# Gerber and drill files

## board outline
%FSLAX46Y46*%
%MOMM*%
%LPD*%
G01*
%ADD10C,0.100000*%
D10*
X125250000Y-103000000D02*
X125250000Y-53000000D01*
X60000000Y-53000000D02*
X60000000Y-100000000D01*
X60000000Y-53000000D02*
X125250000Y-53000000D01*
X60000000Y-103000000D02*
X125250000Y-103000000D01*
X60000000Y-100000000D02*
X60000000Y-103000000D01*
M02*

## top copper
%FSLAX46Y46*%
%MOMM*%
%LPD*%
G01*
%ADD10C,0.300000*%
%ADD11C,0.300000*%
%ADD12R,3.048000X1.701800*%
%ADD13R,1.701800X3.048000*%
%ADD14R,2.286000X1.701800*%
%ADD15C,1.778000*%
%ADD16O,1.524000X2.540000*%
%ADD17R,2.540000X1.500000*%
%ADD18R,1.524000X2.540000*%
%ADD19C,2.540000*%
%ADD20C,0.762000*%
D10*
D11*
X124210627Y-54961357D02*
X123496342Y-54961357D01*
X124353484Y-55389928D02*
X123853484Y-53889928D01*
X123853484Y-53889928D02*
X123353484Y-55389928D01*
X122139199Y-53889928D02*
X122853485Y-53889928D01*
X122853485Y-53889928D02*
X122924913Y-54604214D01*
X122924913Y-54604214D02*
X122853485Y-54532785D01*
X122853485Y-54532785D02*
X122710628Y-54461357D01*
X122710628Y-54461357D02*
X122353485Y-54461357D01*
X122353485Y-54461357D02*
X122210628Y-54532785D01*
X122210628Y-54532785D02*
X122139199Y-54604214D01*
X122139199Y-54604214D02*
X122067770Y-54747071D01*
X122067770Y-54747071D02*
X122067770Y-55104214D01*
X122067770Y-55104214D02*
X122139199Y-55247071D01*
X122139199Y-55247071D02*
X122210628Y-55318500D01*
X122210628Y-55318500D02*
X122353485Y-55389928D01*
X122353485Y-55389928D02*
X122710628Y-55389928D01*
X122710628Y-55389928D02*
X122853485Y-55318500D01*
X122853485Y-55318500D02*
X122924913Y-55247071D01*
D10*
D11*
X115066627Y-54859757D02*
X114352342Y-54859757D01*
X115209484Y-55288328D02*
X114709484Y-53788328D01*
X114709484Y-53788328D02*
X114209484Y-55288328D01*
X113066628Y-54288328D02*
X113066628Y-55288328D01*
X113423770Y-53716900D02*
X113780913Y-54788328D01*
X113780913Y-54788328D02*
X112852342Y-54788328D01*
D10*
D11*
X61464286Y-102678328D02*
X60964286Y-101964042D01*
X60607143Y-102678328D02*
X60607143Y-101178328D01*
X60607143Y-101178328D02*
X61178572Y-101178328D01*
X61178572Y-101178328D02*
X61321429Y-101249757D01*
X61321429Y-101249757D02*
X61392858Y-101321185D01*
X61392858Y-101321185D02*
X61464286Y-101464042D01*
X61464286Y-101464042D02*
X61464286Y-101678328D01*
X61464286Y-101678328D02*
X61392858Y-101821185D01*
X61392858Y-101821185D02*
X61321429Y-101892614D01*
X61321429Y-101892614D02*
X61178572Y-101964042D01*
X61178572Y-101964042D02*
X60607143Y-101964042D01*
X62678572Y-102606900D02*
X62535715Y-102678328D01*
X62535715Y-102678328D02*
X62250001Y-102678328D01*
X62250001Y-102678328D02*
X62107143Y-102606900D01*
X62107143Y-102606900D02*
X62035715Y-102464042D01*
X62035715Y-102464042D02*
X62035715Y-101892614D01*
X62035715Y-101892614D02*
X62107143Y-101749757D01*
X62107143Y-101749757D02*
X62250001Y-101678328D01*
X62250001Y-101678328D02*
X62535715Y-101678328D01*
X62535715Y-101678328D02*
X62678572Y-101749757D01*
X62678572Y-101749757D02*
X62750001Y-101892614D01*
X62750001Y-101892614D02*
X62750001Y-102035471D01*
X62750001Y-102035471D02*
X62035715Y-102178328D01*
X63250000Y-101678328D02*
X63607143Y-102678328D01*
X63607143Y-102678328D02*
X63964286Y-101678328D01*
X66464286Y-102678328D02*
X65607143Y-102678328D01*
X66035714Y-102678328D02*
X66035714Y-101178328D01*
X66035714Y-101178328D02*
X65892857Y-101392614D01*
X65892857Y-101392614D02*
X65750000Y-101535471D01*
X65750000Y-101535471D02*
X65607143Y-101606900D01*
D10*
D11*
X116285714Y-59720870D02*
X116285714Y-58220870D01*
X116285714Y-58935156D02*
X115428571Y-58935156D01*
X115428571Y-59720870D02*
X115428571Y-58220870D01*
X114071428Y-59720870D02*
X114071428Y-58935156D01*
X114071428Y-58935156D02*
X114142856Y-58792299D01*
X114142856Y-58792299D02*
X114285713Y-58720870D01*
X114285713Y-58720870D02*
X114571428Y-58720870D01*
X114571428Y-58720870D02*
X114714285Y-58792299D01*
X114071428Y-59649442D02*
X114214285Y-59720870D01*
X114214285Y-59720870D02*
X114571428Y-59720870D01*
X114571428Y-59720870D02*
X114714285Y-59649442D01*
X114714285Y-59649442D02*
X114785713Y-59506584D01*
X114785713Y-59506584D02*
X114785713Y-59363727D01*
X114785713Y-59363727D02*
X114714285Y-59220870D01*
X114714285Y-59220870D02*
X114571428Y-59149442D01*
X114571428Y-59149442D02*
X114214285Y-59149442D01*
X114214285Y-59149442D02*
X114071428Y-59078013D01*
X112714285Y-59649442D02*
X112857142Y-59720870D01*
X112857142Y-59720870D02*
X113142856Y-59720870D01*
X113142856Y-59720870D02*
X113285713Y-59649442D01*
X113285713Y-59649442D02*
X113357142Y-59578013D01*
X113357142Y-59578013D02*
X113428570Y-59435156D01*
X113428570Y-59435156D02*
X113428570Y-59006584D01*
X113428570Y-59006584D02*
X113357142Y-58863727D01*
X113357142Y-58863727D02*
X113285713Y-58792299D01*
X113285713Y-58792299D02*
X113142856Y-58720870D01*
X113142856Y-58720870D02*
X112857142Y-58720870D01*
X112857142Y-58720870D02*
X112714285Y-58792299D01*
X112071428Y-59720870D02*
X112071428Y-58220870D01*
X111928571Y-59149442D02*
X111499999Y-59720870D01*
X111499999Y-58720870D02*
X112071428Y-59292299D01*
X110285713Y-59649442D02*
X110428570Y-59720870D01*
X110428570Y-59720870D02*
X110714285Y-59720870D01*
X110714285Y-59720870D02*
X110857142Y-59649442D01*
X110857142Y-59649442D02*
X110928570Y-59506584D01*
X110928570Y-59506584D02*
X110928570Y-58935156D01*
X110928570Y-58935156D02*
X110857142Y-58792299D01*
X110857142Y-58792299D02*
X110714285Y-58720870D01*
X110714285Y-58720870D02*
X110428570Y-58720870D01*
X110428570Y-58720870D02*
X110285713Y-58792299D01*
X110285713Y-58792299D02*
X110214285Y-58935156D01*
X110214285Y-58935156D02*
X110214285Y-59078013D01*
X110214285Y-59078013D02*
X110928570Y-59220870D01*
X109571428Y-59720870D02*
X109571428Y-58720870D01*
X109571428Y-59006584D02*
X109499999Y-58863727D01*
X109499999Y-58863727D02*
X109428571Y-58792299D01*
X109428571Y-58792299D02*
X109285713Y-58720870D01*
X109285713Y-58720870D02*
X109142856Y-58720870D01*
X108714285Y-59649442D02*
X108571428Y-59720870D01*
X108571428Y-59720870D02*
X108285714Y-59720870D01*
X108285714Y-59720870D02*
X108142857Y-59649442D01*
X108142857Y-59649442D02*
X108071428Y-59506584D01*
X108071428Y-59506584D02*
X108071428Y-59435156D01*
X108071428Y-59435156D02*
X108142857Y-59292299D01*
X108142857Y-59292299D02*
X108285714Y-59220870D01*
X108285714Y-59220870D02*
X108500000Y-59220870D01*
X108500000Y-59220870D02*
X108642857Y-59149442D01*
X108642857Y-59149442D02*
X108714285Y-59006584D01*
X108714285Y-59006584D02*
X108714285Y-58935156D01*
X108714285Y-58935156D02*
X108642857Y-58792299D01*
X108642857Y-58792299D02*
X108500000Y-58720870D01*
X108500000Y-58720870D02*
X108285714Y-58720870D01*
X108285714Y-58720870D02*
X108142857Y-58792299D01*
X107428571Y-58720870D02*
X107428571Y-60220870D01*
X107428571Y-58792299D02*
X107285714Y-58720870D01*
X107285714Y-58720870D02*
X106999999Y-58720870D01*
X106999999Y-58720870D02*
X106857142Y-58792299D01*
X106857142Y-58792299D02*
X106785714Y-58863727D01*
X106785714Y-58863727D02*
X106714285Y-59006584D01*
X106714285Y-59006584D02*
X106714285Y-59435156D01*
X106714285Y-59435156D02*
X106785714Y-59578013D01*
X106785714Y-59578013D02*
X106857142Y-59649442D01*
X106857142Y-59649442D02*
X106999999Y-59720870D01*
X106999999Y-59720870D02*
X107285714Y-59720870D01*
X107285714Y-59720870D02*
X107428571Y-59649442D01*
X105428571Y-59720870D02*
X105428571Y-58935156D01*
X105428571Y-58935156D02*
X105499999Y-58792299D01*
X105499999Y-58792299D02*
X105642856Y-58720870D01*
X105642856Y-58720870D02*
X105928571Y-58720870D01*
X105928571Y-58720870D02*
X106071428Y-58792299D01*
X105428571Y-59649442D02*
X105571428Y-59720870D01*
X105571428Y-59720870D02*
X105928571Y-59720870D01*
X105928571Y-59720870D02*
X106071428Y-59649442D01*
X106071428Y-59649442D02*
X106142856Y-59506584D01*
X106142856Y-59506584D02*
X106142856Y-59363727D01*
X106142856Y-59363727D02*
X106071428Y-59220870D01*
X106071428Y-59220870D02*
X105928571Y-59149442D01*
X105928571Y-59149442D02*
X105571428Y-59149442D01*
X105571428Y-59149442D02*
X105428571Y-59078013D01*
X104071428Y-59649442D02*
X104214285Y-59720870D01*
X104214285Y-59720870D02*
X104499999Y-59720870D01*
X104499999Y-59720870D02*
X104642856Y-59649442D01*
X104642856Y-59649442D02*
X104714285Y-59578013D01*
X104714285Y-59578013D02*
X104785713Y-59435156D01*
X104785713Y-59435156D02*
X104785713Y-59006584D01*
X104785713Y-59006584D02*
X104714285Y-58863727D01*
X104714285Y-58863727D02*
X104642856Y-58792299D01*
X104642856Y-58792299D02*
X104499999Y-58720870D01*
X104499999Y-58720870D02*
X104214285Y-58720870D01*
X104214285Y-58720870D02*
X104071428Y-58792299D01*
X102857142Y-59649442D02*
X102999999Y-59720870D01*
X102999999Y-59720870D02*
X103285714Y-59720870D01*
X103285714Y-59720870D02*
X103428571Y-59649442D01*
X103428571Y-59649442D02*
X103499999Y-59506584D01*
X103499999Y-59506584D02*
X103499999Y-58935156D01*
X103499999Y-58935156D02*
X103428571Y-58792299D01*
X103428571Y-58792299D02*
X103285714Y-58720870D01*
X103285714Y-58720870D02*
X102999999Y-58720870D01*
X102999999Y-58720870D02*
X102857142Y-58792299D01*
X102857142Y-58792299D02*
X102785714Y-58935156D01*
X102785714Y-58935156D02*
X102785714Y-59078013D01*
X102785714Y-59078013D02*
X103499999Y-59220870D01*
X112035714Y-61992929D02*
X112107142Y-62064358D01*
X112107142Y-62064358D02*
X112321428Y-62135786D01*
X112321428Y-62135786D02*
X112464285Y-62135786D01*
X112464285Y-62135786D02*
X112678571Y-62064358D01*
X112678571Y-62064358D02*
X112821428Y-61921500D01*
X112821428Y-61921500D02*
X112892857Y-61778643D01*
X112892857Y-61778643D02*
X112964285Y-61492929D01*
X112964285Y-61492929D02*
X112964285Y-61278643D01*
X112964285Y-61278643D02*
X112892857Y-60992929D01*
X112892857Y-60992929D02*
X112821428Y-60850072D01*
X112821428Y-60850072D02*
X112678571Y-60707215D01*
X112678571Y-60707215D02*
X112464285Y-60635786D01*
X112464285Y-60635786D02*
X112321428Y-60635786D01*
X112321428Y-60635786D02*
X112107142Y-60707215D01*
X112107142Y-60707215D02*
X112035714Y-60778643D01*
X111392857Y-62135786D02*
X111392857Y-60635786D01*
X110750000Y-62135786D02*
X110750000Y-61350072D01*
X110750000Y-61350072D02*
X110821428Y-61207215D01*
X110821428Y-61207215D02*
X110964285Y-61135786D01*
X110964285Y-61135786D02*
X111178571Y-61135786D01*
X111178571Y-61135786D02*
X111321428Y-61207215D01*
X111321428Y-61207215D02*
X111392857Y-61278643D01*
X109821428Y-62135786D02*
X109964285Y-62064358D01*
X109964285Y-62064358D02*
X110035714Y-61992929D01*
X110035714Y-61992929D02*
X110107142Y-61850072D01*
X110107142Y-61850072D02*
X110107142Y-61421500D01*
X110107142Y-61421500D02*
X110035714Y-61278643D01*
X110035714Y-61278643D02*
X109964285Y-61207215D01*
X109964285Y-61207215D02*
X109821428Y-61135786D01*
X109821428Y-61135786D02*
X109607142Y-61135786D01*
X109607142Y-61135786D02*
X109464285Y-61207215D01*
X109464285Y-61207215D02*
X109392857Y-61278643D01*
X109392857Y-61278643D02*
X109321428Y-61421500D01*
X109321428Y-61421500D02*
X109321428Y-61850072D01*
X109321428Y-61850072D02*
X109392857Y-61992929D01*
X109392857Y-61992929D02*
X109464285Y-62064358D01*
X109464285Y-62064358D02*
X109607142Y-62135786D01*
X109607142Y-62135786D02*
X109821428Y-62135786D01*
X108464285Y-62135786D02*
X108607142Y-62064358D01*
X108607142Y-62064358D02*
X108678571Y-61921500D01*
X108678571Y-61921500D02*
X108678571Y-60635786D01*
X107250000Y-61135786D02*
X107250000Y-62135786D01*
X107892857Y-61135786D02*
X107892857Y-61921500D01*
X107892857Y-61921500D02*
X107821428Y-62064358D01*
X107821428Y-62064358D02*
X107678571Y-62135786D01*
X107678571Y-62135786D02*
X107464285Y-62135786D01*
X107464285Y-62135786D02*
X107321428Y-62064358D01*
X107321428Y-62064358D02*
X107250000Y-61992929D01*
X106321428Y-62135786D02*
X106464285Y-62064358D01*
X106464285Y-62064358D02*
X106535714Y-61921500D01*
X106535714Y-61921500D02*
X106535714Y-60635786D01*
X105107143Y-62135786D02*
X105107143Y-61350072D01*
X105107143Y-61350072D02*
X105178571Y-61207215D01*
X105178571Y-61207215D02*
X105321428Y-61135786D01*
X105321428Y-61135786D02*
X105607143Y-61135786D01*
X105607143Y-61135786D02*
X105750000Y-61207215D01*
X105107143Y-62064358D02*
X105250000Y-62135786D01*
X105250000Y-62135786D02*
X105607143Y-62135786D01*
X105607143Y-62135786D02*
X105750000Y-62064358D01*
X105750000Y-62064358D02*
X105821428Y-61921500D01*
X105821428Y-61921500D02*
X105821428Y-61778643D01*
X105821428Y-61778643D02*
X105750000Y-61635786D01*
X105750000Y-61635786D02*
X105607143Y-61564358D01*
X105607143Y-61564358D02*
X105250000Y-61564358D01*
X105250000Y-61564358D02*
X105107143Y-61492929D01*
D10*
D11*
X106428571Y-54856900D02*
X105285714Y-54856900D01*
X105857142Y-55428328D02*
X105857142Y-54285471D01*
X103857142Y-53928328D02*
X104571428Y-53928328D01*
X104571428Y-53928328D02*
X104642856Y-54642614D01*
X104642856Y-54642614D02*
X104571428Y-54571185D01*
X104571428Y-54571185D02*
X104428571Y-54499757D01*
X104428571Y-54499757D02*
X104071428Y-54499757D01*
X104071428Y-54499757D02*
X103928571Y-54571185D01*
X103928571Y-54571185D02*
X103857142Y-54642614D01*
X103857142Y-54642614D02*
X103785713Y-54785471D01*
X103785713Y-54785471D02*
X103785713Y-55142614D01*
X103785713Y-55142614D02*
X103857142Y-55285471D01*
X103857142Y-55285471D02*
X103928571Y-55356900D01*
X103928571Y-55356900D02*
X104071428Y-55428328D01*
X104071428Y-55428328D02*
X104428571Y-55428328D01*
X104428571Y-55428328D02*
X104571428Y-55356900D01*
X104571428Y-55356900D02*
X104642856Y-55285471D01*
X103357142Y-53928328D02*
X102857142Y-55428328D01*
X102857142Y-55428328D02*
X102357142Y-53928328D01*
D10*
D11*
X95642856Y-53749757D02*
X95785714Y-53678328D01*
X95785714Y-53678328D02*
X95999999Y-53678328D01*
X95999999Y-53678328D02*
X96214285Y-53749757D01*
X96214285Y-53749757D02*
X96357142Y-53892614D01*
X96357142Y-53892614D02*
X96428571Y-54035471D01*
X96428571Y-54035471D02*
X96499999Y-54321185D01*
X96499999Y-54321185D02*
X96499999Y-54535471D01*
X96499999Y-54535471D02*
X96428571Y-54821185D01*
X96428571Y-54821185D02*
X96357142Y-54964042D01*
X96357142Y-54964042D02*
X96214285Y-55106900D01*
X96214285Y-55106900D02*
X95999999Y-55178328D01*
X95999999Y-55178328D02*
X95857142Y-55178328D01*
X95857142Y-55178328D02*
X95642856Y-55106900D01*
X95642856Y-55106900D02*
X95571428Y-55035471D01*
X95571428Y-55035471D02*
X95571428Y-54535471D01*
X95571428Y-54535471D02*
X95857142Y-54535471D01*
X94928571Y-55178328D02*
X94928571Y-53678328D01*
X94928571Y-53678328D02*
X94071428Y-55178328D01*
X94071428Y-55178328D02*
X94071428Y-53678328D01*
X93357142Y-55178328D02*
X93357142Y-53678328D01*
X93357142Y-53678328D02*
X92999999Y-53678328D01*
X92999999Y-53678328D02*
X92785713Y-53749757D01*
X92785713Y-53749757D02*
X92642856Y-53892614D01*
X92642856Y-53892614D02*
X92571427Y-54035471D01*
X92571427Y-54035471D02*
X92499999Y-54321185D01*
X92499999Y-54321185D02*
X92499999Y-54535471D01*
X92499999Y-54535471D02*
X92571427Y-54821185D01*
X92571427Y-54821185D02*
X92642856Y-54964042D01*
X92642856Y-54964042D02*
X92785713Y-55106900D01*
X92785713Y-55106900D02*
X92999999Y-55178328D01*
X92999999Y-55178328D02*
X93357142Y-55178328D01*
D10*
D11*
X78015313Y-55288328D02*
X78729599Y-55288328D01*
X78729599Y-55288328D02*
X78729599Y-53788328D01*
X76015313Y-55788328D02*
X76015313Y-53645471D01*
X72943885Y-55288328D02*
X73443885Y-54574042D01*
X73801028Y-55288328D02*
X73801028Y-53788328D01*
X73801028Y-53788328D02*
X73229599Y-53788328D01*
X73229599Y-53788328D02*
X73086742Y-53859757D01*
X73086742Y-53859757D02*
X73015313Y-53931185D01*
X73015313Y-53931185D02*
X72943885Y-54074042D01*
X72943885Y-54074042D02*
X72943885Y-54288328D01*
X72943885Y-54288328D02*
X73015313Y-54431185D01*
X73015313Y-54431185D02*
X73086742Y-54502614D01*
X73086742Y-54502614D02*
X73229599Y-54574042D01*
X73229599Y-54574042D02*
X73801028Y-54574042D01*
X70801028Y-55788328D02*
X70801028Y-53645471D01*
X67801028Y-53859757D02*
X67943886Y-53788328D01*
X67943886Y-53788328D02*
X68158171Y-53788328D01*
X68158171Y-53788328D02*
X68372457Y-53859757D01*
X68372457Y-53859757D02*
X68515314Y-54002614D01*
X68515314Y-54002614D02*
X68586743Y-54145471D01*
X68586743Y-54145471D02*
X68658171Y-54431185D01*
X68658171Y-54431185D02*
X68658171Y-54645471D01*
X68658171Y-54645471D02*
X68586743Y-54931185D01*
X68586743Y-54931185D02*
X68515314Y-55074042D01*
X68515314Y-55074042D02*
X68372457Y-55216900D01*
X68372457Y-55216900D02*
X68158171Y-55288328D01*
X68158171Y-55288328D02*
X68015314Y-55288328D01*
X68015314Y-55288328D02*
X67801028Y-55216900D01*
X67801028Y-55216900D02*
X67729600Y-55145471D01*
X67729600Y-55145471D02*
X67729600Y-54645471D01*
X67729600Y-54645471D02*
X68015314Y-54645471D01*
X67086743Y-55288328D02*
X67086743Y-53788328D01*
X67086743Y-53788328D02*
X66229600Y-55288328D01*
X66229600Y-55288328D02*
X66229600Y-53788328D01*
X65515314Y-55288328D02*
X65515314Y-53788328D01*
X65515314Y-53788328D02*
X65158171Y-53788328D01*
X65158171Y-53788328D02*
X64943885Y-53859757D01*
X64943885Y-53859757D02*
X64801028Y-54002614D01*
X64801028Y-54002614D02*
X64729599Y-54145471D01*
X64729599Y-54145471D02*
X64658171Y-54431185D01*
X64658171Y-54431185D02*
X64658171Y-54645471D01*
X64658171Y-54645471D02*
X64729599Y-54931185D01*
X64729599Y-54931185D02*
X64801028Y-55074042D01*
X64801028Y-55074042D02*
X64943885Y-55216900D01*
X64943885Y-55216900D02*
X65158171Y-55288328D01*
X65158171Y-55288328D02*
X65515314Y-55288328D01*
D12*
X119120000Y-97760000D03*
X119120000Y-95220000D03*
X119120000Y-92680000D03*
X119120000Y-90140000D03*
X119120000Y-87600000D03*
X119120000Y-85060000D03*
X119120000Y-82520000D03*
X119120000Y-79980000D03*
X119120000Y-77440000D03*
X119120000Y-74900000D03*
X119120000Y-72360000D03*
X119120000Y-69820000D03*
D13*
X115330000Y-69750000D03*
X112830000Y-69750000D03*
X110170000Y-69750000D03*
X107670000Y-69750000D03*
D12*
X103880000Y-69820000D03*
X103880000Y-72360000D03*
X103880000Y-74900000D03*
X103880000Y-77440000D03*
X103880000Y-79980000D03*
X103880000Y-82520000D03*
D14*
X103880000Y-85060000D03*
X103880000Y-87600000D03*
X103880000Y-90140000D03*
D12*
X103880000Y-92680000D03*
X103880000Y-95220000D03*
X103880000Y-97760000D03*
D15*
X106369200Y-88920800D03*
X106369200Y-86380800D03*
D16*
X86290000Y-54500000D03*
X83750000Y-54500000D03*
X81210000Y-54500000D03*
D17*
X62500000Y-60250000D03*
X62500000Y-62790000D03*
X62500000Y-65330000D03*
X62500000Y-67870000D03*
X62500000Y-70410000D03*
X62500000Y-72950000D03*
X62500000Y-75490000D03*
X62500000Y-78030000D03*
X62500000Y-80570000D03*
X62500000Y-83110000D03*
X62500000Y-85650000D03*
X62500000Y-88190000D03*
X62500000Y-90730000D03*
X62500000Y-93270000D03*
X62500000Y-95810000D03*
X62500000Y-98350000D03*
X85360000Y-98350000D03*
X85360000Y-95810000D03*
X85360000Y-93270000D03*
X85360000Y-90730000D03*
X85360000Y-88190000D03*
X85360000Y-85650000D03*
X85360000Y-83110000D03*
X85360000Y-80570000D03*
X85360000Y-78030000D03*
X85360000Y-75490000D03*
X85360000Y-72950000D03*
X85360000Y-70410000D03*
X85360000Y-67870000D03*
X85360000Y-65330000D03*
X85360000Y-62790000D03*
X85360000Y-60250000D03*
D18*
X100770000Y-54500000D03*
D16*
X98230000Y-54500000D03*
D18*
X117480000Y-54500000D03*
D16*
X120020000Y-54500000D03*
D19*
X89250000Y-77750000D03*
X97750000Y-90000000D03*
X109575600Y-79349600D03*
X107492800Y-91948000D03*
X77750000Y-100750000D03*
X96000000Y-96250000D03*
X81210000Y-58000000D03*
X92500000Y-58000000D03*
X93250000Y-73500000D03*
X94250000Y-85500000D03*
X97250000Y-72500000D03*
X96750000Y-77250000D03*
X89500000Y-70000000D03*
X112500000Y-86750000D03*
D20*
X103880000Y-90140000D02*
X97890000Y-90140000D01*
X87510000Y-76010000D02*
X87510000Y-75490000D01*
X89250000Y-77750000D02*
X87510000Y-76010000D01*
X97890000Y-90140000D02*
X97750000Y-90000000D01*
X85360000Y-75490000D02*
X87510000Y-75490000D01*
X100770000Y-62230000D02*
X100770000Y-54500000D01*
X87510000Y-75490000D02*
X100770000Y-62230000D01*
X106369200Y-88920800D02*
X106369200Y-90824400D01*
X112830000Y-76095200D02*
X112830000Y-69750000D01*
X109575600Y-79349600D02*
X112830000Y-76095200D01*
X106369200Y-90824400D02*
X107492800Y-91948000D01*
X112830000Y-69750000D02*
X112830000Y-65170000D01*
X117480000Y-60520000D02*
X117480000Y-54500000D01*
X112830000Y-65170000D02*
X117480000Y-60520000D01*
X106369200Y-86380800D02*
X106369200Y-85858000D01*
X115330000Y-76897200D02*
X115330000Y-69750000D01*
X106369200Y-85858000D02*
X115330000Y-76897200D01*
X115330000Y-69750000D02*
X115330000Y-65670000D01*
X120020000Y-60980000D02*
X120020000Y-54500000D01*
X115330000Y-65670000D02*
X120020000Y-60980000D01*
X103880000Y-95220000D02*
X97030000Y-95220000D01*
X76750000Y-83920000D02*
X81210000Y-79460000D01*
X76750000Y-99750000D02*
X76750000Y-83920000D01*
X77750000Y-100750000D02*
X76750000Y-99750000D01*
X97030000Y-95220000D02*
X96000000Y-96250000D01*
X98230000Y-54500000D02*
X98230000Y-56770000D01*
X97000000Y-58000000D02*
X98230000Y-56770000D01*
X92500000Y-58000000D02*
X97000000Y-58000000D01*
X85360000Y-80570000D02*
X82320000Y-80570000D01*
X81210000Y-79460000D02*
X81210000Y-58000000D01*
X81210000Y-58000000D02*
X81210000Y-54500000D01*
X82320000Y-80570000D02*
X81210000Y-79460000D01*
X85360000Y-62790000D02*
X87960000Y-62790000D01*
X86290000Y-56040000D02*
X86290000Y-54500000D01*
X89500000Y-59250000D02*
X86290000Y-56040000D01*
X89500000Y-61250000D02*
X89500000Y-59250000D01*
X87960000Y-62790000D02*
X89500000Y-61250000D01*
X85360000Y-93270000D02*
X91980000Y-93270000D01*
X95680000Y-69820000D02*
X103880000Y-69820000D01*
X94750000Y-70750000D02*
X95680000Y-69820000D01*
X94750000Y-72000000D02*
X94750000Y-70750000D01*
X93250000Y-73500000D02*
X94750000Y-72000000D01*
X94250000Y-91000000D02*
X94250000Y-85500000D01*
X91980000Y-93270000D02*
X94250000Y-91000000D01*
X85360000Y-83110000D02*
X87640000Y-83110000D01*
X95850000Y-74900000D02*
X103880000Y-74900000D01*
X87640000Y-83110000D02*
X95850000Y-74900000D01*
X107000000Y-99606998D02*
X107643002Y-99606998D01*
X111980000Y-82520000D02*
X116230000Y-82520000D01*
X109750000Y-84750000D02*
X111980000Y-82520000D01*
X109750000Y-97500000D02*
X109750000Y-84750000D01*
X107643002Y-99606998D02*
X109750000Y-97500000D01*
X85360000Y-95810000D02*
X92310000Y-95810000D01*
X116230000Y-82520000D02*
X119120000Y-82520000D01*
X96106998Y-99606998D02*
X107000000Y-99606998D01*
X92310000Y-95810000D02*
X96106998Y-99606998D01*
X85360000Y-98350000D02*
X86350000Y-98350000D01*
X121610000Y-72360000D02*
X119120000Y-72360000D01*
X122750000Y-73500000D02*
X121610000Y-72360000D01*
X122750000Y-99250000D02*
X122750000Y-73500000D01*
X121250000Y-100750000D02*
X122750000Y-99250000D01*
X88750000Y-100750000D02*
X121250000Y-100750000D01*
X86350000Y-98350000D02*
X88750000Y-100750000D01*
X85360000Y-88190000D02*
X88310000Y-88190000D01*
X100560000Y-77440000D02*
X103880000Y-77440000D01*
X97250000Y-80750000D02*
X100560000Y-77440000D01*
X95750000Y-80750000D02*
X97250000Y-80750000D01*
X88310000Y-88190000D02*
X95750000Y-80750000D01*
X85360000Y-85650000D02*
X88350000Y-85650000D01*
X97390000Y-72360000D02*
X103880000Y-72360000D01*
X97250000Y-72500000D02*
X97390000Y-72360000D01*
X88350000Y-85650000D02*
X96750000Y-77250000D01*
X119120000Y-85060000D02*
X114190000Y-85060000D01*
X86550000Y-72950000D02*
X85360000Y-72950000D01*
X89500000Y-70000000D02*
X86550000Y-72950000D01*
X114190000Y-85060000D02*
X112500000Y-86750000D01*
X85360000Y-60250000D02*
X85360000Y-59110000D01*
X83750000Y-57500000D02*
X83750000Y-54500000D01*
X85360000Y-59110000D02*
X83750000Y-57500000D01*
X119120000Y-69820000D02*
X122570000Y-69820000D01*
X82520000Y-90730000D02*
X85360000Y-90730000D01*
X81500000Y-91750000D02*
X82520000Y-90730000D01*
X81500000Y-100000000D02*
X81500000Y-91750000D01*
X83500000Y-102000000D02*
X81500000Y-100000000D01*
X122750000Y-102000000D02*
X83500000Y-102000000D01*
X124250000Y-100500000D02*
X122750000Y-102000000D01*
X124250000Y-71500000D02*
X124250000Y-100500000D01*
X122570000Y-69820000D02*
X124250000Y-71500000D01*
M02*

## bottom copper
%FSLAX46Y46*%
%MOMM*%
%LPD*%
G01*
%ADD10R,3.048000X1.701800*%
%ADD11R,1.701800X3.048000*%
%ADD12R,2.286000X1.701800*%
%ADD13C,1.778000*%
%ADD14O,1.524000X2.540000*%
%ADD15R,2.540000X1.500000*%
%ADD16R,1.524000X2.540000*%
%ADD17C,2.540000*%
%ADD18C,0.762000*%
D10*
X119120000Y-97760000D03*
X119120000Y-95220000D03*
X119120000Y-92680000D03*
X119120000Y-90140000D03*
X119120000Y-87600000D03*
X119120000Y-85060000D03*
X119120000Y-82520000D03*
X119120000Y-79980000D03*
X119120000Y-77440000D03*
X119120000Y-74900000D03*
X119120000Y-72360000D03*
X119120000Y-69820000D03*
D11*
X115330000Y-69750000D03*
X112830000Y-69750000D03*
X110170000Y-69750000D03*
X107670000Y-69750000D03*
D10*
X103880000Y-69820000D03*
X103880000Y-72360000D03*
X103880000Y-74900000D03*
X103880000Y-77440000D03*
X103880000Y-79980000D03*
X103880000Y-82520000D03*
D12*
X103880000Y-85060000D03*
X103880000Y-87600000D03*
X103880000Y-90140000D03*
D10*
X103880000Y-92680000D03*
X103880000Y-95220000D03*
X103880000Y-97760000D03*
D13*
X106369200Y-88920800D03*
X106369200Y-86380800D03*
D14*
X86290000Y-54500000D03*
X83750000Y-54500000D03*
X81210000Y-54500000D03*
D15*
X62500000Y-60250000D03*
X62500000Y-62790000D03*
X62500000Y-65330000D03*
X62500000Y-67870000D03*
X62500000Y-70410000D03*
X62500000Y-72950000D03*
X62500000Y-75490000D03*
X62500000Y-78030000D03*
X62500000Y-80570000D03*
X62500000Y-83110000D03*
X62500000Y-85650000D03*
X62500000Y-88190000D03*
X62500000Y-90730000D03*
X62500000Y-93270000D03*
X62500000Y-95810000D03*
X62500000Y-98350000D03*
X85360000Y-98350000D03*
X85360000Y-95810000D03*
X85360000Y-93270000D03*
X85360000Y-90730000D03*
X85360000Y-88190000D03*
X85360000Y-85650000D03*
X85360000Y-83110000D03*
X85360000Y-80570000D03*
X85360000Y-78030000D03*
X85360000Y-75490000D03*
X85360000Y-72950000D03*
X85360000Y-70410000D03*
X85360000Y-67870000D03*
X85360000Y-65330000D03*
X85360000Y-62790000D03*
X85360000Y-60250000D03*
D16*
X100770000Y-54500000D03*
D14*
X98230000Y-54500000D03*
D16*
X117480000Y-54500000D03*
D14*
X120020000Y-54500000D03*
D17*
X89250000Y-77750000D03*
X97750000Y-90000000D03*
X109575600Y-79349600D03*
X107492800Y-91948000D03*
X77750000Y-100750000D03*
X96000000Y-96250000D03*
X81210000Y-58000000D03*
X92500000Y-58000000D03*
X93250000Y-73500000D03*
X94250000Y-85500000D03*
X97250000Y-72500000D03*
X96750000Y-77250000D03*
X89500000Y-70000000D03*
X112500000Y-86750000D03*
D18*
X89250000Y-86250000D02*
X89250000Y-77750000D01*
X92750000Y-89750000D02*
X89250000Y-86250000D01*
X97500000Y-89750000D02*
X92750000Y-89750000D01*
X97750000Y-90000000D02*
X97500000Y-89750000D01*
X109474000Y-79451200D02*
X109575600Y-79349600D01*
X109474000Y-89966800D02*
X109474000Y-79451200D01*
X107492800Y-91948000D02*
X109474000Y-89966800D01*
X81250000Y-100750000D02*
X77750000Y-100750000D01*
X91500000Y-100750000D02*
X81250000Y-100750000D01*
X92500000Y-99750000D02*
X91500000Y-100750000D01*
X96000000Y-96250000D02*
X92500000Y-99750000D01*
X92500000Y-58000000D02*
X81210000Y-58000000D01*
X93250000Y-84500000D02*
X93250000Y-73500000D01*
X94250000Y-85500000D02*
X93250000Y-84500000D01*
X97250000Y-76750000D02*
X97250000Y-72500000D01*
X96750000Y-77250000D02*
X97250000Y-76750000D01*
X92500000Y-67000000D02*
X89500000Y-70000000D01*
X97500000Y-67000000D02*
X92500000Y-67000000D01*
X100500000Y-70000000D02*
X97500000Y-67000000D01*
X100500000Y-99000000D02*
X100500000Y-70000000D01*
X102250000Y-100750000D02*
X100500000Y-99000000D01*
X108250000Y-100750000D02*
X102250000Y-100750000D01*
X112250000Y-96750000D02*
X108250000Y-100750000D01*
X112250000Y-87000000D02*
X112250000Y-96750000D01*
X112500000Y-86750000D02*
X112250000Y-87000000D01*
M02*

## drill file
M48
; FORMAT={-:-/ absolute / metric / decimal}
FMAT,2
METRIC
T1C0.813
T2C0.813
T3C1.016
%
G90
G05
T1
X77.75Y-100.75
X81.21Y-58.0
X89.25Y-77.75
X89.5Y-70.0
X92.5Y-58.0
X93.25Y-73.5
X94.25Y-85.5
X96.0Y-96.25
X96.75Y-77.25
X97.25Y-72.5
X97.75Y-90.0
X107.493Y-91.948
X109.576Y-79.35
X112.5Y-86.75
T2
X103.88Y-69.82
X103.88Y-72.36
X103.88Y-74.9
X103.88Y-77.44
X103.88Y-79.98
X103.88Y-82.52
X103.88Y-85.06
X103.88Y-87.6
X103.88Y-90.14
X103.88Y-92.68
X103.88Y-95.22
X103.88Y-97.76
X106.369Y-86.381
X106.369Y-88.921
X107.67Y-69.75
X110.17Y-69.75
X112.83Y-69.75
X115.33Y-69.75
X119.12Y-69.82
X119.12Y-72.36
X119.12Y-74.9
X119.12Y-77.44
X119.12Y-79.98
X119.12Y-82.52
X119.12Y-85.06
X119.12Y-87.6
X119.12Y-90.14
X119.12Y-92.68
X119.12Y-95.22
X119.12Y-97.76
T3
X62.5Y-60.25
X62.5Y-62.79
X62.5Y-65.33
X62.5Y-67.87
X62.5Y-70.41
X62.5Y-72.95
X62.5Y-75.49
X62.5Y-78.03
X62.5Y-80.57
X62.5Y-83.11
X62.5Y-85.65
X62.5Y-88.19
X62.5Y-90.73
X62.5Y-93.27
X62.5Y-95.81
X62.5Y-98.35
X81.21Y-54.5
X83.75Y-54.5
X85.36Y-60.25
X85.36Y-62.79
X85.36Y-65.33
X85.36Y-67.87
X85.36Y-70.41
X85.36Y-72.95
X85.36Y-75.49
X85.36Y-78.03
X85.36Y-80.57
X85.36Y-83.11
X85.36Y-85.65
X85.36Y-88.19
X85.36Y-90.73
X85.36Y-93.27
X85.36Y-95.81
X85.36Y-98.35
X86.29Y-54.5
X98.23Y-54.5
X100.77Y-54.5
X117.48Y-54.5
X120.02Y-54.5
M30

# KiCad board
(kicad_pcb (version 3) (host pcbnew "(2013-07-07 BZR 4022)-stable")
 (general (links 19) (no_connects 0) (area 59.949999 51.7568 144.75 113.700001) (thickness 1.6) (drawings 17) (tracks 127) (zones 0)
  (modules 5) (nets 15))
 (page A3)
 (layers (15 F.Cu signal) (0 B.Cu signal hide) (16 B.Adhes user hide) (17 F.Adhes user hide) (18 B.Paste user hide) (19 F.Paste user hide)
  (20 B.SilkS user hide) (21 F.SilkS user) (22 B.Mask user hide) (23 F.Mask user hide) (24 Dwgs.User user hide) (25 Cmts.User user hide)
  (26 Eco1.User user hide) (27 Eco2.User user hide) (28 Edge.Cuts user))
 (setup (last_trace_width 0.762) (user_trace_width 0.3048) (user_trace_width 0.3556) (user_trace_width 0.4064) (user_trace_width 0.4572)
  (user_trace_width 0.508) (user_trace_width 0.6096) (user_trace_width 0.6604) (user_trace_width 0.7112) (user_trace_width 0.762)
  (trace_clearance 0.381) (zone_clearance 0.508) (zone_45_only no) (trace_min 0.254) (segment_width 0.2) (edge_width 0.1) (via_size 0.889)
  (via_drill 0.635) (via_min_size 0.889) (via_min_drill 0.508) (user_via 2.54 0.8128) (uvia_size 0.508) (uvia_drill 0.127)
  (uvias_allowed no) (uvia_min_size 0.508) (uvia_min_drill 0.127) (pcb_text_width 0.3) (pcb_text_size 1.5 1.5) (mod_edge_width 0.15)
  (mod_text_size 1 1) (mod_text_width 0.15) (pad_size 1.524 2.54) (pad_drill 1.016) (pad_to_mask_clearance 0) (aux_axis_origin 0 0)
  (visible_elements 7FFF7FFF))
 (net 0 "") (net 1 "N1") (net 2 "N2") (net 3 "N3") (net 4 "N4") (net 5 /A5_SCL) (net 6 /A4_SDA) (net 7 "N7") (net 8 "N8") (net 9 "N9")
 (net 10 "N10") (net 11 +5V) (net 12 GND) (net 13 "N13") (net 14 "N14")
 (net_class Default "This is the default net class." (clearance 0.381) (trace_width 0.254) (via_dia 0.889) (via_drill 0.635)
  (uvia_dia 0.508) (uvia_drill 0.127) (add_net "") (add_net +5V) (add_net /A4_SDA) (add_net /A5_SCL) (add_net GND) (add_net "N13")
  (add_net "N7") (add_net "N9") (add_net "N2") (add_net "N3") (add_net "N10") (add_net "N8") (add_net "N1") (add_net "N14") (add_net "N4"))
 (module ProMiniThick (layer F.Cu) (at 111.5 81.25 90)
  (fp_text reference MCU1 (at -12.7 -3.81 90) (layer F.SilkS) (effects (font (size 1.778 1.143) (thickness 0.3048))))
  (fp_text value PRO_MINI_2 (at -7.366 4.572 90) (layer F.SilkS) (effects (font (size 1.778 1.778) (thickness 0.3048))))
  (pad 1 thru_hole rect (at -16.51 7.62 90) (size 1.7018 3.048) (drill 0.8128) (layers *.Cu *.Mask F.SilkS))
  (pad 2 thru_hole rect (at -13.97 7.62 90) (size 1.7018 3.048) (drill 0.8128) (layers *.Cu *.Mask F.SilkS))
  (pad 3 thru_hole rect (at -11.43 7.62 90) (size 1.7018 3.048) (drill 0.8128) (layers *.Cu *.Mask F.SilkS))
  (pad 4 thru_hole rect (at -8.89 7.62 90) (size 1.7018 3.048) (drill 0.8128) (layers *.Cu *.Mask F.SilkS))
  (pad 5 thru_hole rect (at -6.35 7.62 90) (size 1.7018 3.048) (drill 0.8128) (layers *.Cu *.Mask F.SilkS))
  (pad 6 thru_hole rect (at -3.81 7.62 90) (size 1.7018 3.048) (drill 0.8128) (layers *.Cu *.Mask F.SilkS) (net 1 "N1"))
  (pad 7 thru_hole rect (at -1.27 7.62 90) (size 1.7018 3.048) (drill 0.8128) (layers *.Cu *.Mask F.SilkS) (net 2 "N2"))
  (pad 8 thru_hole rect (at 1.27 7.62 90) (size 1.7018 3.048) (drill 0.8128) (layers *.Cu *.Mask F.SilkS))
  (pad 9 thru_hole rect (at 3.81 7.62 90) (size 1.7018 3.048) (drill 0.8128) (layers *.Cu *.Mask F.SilkS))
  (pad 10 thru_hole rect (at 6.35 7.62 90) (size 1.7018 3.048) (drill 0.8128) (layers *.Cu *.Mask F.SilkS))
  (pad 11 thru_hole rect (at 8.89 7.62 90) (size 1.7018 3.048) (drill 0.8128) (layers *.Cu *.Mask F.SilkS) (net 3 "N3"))
  (pad 12 thru_hole rect (at 11.43 7.62 90) (size 1.7018 3.048) (drill 0.8128) (layers *.Cu *.Mask F.SilkS) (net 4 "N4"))
  (pad 13 thru_hole rect (at 11.5 3.83 90) (size 3.048 1.7018) (drill 0.8128) (layers *.Cu *.Mask F.SilkS) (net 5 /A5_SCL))
  (pad 14 thru_hole rect (at 11.5 1.33 90) (size 3.048 1.7018) (drill 0.8128) (layers *.Cu *.Mask F.SilkS) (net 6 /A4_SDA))
  (pad 15 thru_hole rect (at 11.5 -1.33 90) (size 3.048 1.7018) (drill 0.8128) (layers *.Cu *.Mask F.SilkS))
  (pad 16 thru_hole rect (at 11.5 -3.83 90) (size 3.048 1.7018) (drill 0.8128) (layers *.Cu *.Mask F.SilkS))
  (pad 17 thru_hole rect (at 11.43 -7.62 90) (size 1.7018 3.048) (drill 0.8128) (layers *.Cu *.Mask F.SilkS) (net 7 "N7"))
  (pad 18 thru_hole rect (at 8.89 -7.62 90) (size 1.7018 3.048) (drill 0.8128) (layers *.Cu *.Mask F.SilkS) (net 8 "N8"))
  (pad 19 thru_hole rect (at 6.35 -7.62 90) (size 1.7018 3.048) (drill 0.8128) (layers *.Cu *.Mask F.SilkS) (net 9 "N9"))
  (pad 20 thru_hole rect (at 3.81 -7.62 90) (size 1.7018 3.048) (drill 0.8128) (layers *.Cu *.Mask F.SilkS) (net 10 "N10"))
  (pad 21 thru_hole rect (at 1.27 -7.62 90) (size 1.7018 3.048) (drill 0.8128) (layers *.Cu *.Mask F.SilkS))
  (pad 22 thru_hole rect (at -1.27 -7.62 90) (size 1.7018 3.048) (drill 0.8128) (layers *.Cu *.Mask F.SilkS))
  (pad 23 thru_hole rect (at -3.81 -7.62 90) (size 1.7018 2.286) (drill 0.8128) (layers *.Cu *.Mask F.SilkS))
  (pad 24 thru_hole rect (at -6.35 -7.62 90) (size 1.7018 2.286) (drill 0.8128) (layers *.Cu *.Mask F.SilkS))
  (pad 25 thru_hole rect (at -8.89 -7.62 90) (size 1.7018 2.286) (drill 0.8128) (layers *.Cu *.Mask F.SilkS) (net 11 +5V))
  (pad 26 thru_hole rect (at -11.43 -7.62 90) (size 1.7018 3.048) (drill 0.8128) (layers *.Cu *.Mask F.SilkS))
  (pad 27 thru_hole rect (at -13.97 -7.62 90) (size 1.7018 3.048) (drill 0.8128) (layers *.Cu *.Mask F.SilkS) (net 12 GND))
  (pad 28 thru_hole rect (at -16.51 -7.62 90) (size 1.7018 3.048) (drill 0.8128) (layers *.Cu *.Mask F.SilkS))
  (pad 14 thru_hole circle (at -7.6708 -5.1308 90) (size 1.778 1.778) (drill 0.8128) (layers *.Cu *.Mask F.SilkS) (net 6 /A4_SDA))
  (pad 13 thru_hole circle (at -5.1308 -5.1308 90) (size 1.778 1.778) (drill 0.8128) (layers *.Cu *.Mask F.SilkS) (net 5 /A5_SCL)))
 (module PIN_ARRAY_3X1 (layer F.Cu) (at 83.75 54.5 180)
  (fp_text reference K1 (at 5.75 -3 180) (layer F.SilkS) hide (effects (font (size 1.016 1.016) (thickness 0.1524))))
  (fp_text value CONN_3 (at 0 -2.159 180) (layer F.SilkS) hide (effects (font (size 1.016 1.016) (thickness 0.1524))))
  (pad 1 thru_hole oval (at -2.54 0 180) (size 1.524 2.54) (drill 1.016) (layers *.Cu *.Mask F.SilkS) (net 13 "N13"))
  (pad 2 thru_hole oval (at 0 0 180) (size 1.524 2.54) (drill 1.016) (layers *.Cu *.Mask F.SilkS) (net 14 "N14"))
  (pad 3 thru_hole oval (at 2.54 0 180) (size 1.524 2.54) (drill 1.016) (layers *.Cu *.Mask F.SilkS) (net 12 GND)))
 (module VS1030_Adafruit (layer F.Cu) (at 62.5 60.25)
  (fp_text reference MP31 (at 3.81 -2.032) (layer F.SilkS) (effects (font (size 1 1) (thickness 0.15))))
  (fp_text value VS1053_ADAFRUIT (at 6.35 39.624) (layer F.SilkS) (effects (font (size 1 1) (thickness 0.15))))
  (pad 1 thru_hole rect (at 0 0) (size 2.54 1.5) (drill 1.016) (layers *.Cu *.Mask F.SilkS))
  (pad 2 thru_hole rect (at 0 2.54) (size 2.54 1.5) (drill 1.016) (layers *.Cu *.Mask F.SilkS))
  (pad 3 thru_hole rect (at 0 5.08) (size 2.54 1.5) (drill 1.016) (layers *.Cu *.Mask F.SilkS))
  (pad 4 thru_hole rect (at 0 7.62) (size 2.54 1.5) (drill 1.016) (layers *.Cu *.Mask F.SilkS))
  (pad 5 thru_hole rect (at 0 10.16) (size 2.54 1.5) (drill 1.016) (layers *.Cu *.Mask F.SilkS))
  (pad 6 thru_hole rect (at 0 12.7) (size 2.54 1.5) (drill 1.016) (layers *.Cu *.Mask F.SilkS))
  (pad 7 thru_hole rect (at 0 15.24) (size 2.54 1.5) (drill 1.016) (layers *.Cu *.Mask F.SilkS))
  (pad 8 thru_hole rect (at 0 17.78) (size 2.54 1.5) (drill 1.016) (layers *.Cu *.Mask F.SilkS))
  (pad 9 thru_hole rect (at 0 20.32) (size 2.54 1.5) (drill 1.016) (layers *.Cu *.Mask F.SilkS))
  (pad 10 thru_hole rect (at 0 22.86) (size 2.54 1.5) (drill 1.016) (layers *.Cu *.Mask F.SilkS))
  (pad 11 thru_hole rect (at 0 25.4) (size 2.54 1.5) (drill 1.016) (layers *.Cu *.Mask F.SilkS))
  (pad 12 thru_hole rect (at 0 27.94) (size 2.54 1.5) (drill 1.016) (layers *.Cu *.Mask F.SilkS))
  (pad 13 thru_hole rect (at 0 30.48) (size 2.54 1.5) (drill 1.016) (layers *.Cu *.Mask F.SilkS))
  (pad 14 thru_hole rect (at 0 33.02) (size 2.54 1.5) (drill 1.016) (layers *.Cu *.Mask F.SilkS))
  (pad 15 thru_hole rect (at 0 35.56) (size 2.54 1.5) (drill 1.016) (layers *.Cu *.Mask F.SilkS))
  (pad 16 thru_hole rect (at 0 38.1) (size 2.54 1.5) (drill 1.016) (layers *.Cu *.Mask F.SilkS))
  (pad 17 thru_hole rect (at 22.86 38.1) (size 2.54 1.5) (drill 1.016) (layers *.Cu *.Mask F.SilkS) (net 3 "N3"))
  (pad 18 thru_hole rect (at 22.86 35.56) (size 2.54 1.5) (drill 1.016) (layers *.Cu *.Mask F.SilkS) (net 2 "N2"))
  (pad 19 thru_hole rect (at 22.86 33.02) (size 2.54 1.5) (drill 1.016) (layers *.Cu *.Mask F.SilkS) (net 7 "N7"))
  (pad 20 thru_hole rect (at 22.86 30.48) (size 2.54 1.5) (drill 1.016) (layers *.Cu *.Mask F.SilkS) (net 4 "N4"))
  (pad 21 thru_hole rect (at 22.86 27.94) (size 2.54 1.5) (drill 1.016) (layers *.Cu *.Mask F.SilkS) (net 10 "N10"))
  (pad 22 thru_hole rect (at 22.86 25.4) (size 2.54 1.5) (drill 1.016) (layers *.Cu *.Mask F.SilkS) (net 8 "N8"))
  (pad 23 thru_hole rect (at 22.86 22.86) (size 2.54 1.5) (drill 1.016) (layers *.Cu *.Mask F.SilkS) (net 9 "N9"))
  (pad 24 thru_hole rect (at 22.86 20.32) (size 2.54 1.5) (drill 1.016) (layers *.Cu *.Mask F.SilkS) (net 12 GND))
  (pad 25 thru_hole rect (at 22.86 17.78) (size 2.54 1.5) (drill 1.016) (layers *.Cu *.Mask F.SilkS))
  (pad 26 thru_hole rect (at 22.86 15.24) (size 2.54 1.5) (drill 1.016) (layers *.Cu *.Mask F.SilkS) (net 11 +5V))
  (pad 27 thru_hole rect (at 22.86 12.7) (size 2.54 1.5) (drill 1.016) (layers *.Cu *.Mask F.SilkS) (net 1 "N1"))
  (pad 28 thru_hole rect (at 22.86 10.16) (size 2.54 1.5) (drill 1.016) (layers *.Cu *.Mask F.SilkS))
  (pad 29 thru_hole rect (at 22.86 7.62) (size 2.54 1.5) (drill 1.016) (layers *.Cu *.Mask F.SilkS))
  (pad 30 thru_hole rect (at 22.86 5.08) (size 2.54 1.5) (drill 1.016) (layers *.Cu *.Mask F.SilkS))
  (pad 31 thru_hole rect (at 22.86 2.54) (size 2.54 1.5) (drill 1.016) (layers *.Cu *.Mask F.SilkS) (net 13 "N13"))
  (pad 32 thru_hole rect (at 22.86 0) (size 2.54 1.5) (drill 1.016) (layers *.Cu *.Mask F.SilkS) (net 14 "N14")))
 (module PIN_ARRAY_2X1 (layer F.Cu) (at 99.5 54.5 180)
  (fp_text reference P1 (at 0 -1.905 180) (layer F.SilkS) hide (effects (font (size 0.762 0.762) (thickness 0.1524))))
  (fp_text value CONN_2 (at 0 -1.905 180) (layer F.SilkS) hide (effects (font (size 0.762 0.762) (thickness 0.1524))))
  (pad 1 thru_hole rect (at -1.27 0 180) (size 1.524 2.54) (drill 1.016) (layers *.Cu *.Mask F.SilkS) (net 11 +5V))
  (pad 2 thru_hole oval (at 1.27 0 180) (size 1.524 2.54) (drill 1.016) (layers *.Cu *.Mask F.SilkS) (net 12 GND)))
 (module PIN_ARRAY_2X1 (layer F.Cu) (at 118.75 54.5)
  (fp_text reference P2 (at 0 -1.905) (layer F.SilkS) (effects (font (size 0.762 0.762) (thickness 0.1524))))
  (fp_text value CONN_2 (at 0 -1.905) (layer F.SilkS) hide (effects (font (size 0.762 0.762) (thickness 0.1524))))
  (pad 1 thru_hole rect (at -1.27 0) (size 1.524 2.54) (drill 1.016) (layers *.Cu *.Mask F.SilkS) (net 6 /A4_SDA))
  (pad 2 thru_hole oval (at 1.27 0) (size 1.524 2.54) (drill 1.016) (layers *.Cu *.Mask F.SilkS) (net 5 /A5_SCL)))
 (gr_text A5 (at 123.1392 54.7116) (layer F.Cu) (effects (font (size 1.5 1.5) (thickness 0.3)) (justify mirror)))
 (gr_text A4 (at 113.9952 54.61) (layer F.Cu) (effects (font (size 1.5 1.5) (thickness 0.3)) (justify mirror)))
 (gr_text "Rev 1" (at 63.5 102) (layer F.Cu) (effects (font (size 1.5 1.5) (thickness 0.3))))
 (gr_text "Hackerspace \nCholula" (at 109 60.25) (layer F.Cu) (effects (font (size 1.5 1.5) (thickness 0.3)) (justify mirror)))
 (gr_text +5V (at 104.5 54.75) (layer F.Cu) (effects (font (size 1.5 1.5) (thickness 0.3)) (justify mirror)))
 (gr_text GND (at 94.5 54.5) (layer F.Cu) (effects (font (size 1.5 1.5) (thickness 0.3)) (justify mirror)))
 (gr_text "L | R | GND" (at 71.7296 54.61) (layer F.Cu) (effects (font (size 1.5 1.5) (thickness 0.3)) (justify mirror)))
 (gr_line (start 125.25 103) (end 125.25 53) (angle 90) (layer Edge.Cuts) (width 0.1))
 (gr_line (start 60 53) (end 60 100) (angle 90) (layer Edge.Cuts) (width 0.1))
 (gr_line (start 60 53) (end 125.25 53) (angle 90) (layer Edge.Cuts) (width 0.1))
 (gr_line (start 60 103) (end 125.25 103) (angle 90) (layer Edge.Cuts) (width 0.1))
 (gr_line (start 60 100) (end 60 103) (angle 90) (layer Edge.Cuts) (width 0.1))
 (segment (start 103.88 90.14) (end 97.89 90.14) (width 0.762) (layer F.Cu) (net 11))
 (segment (start 87.51 76.01) (end 87.51 75.49) (width 0.762) (layer F.Cu) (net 11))
 (segment (start 89.25 77.75) (end 87.51 76.01) (width 0.762) (layer F.Cu) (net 11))
 (via (at 89.25 77.75) (size 2.54) (drill 0.8128) (layers F.Cu B.Cu) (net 11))
 (segment (start 89.25 86.25) (end 89.25 77.75) (width 0.762) (layer B.Cu) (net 11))
 (segment (start 92.75 89.75) (end 89.25 86.25) (width 0.762) (layer B.Cu) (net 11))
 (segment (start 97.5 89.75) (end 92.75 89.75) (width 0.762) (layer B.Cu) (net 11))
 (segment (start 97.75 90) (end 97.5 89.75) (width 0.762) (layer B.Cu) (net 11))
 (via (at 97.75 90) (size 2.54) (drill 0.8128) (layers F.Cu B.Cu) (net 11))
 (segment (start 97.89 90.14) (end 97.75 90) (width 0.762) (layer F.Cu) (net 11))
 (segment (start 85.36 75.49) (end 87.51 75.49) (width 0.762) (layer F.Cu) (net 11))
 (segment (start 100.77 62.23) (end 100.77 54.5) (width 0.762) (layer F.Cu) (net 11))
 (segment (start 87.51 75.49) (end 100.77 62.23) (width 0.762) (layer F.Cu) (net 11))
 (segment (start 106.3692 88.9208) (end 106.3692 90.8244) (width 0.762) (layer F.Cu) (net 6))
 (segment (start 112.83 76.0952) (end 112.83 69.75) (width 0.762) (layer F.Cu) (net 6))
 (segment (start 109.5756 79.3496) (end 112.83 76.0952) (width 0.762) (layer F.Cu) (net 6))
 (via (at 109.5756 79.3496) (size 2.54) (drill 0.8128) (layers F.Cu B.Cu) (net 6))
 (segment (start 109.474 79.4512) (end 109.5756 79.3496) (width 0.762) (layer B.Cu) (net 6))
 (segment (start 109.474 89.9668) (end 109.474 79.4512) (width 0.762) (layer B.Cu) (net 6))
 (segment (start 107.4928 91.948) (end 109.474 89.9668) (width 0.762) (layer B.Cu) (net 6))
 (via (at 107.4928 91.948) (size 2.54) (drill 0.8128) (layers F.Cu B.Cu) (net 6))
 (segment (start 106.3692 90.8244) (end 107.4928 91.948) (width 0.762) (layer F.Cu) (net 6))
 (segment (start 112.83 69.75) (end 112.83 65.17) (width 0.762) (layer F.Cu) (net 6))
 (segment (start 117.48 60.52) (end 117.48 54.5) (width 0.762) (layer F.Cu) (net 6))
 (segment (start 112.83 65.17) (end 117.48 60.52) (width 0.762) (layer F.Cu) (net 6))
 (segment (start 106.3692 86.3808) (end 106.3692 85.858) (width 0.762) (layer F.Cu) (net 5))
 (segment (start 115.33 76.8972) (end 115.33 69.75) (width 0.762) (layer F.Cu) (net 5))
 (segment (start 106.3692 85.858) (end 115.33 76.8972) (width 0.762) (layer F.Cu) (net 5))
 (segment (start 115.33 69.75) (end 115.33 65.67) (width 0.762) (layer F.Cu) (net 5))
 (segment (start 120.02 60.98) (end 120.02 54.5) (width 0.762) (layer F.Cu) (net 5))
 (segment (start 115.33 65.67) (end 120.02 60.98) (width 0.762) (layer F.Cu) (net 5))
 (segment (start 103.88 95.22) (end 97.03 95.22) (width 0.762) (layer F.Cu) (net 12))
 (segment (start 76.75 83.92) (end 81.21 79.46) (width 0.762) (layer F.Cu) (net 12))
 (segment (start 76.75 99.75) (end 76.75 83.92) (width 0.762) (layer F.Cu) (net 12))
 (segment (start 77.75 100.75) (end 76.75 99.75) (width 0.762) (layer F.Cu) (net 12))
 (via (at 77.75 100.75) (size 2.54) (drill 0.8128) (layers F.Cu B.Cu) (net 12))
 (segment (start 81.25 100.75) (end 77.75 100.75) (width 0.762) (layer B.Cu) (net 12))
 (segment (start 91.5 100.75) (end 81.25 100.75) (width 0.762) (layer B.Cu) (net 12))
 (segment (start 92.5 99.75) (end 91.5 100.75) (width 0.762) (layer B.Cu) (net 12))
 (segment (start 96 96.25) (end 92.5 99.75) (width 0.762) (layer B.Cu) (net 12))
 (via (at 96 96.25) (size 2.54) (drill 0.8128) (layers F.Cu B.Cu) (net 12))
 (segment (start 97.03 95.22) (end 96 96.25) (width 0.762) (layer F.Cu) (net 12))
 (via (at 81.21 58) (size 2.54) (drill 0.8128) (layers F.Cu B.Cu) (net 12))
 (segment (start 98.23 54.5) (end 98.23 56.77) (width 0.762) (layer F.Cu) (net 12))
 (segment (start 97 58) (end 98.23 56.77) (width 0.762) (layer F.Cu) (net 12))
 (segment (start 92.5 58) (end 97 58) (width 0.762) (layer F.Cu) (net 12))
 (via (at 92.5 58) (size 2.54) (drill 0.8128) (layers F.Cu B.Cu) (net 12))
 (segment (start 92.5 58) (end 81.21 58) (width 0.762) (layer B.Cu) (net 12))
 (segment (start 85.36 80.57) (end 82.32 80.57) (width 0.762) (layer F.Cu) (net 12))
 (segment (start 81.21 79.46) (end 81.21 58) (width 0.762) (layer F.Cu) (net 12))
 (segment (start 81.21 58) (end 81.21 54.5) (width 0.762) (layer F.Cu) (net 12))
 (segment (start 82.32 80.57) (end 81.21 79.46) (width 0.762) (layer F.Cu) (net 12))
 (segment (start 85.36 62.79) (end 87.96 62.79) (width 0.762) (layer F.Cu) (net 13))
 (segment (start 86.29 56.04) (end 86.29 54.5) (width 0.762) (layer F.Cu) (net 13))
 (segment (start 89.5 59.25) (end 86.29 56.04) (width 0.762) (layer F.Cu) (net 13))
 (segment (start 89.5 61.25) (end 89.5 59.25) (width 0.762) (layer F.Cu) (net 13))
 (segment (start 87.96 62.79) (end 89.5 61.25) (width 0.762) (layer F.Cu) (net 13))
 (segment (start 85.36 93.27) (end 91.98 93.27) (width 0.762) (layer F.Cu) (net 7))
 (segment (start 95.68 69.82) (end 103.88 69.82) (width 0.762) (layer F.Cu) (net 7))
 (segment (start 94.75 70.75) (end 95.68 69.82) (width 0.762) (layer F.Cu) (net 7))
 (segment (start 94.75 72) (end 94.75 70.75) (width 0.762) (layer F.Cu) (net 7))
 (segment (start 93.25 73.5) (end 94.75 72) (width 0.762) (layer F.Cu) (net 7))
 (via (at 93.25 73.5) (size 2.54) (drill 0.8128) (layers F.Cu B.Cu) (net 7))
 (segment (start 93.25 84.5) (end 93.25 73.5) (width 0.762) (layer B.Cu) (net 7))
 (segment (start 94.25 85.5) (end 93.25 84.5) (width 0.762) (layer B.Cu) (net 7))
 (via (at 94.25 85.5) (size 2.54) (drill 0.8128) (layers F.Cu B.Cu) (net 7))
 (segment (start 94.25 91) (end 94.25 85.5) (width 0.762) (layer F.Cu) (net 7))
 (segment (start 91.98 93.27) (end 94.25 91) (width 0.762) (layer F.Cu) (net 7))
 (segment (start 85.36 83.11) (end 87.64 83.11) (width 0.762) (layer F.Cu) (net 9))
 (segment (start 95.85 74.9) (end 103.88 74.9) (width 0.762) (layer F.Cu) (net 9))
 (segment (start 87.64 83.11) (end 95.85 74.9) (width 0.762) (layer F.Cu) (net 9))
 (segment (start 107 99.606998) (end 107.643002 99.606998) (width 0.762) (layer F.Cu) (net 2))
 (segment (start 111.98 82.52) (end 116.23 82.52) (width 0.762) (layer F.Cu) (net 2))
 (segment (start 109.75 84.75) (end 111.98 82.52) (width 0.762) (layer F.Cu) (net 2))
 (segment (start 109.75 97.5) (end 109.75 84.75) (width 0.762) (layer F.Cu) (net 2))
 (segment (start 107.643002 99.606998) (end 109.75 97.5) (width 0.762) (layer F.Cu) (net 2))
 (segment (start 85.36 95.81) (end 92.31 95.81) (width 0.762) (layer F.Cu) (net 2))
 (segment (start 116.23 82.52) (end 119.12 82.52) (width 0.762) (layer F.Cu) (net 2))
 (segment (start 96.106998 99.606998) (end 107 99.606998) (width 0.762) (layer F.Cu) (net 2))
 (segment (start 92.31 95.81) (end 96.106998 99.606998) (width 0.762) (layer F.Cu) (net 2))
 (segment (start 85.36 98.35) (end 86.35 98.35) (width 0.762) (layer F.Cu) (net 3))
 (segment (start 121.61 72.36) (end 119.12 72.36) (width 0.762) (layer F.Cu) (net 3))
 (segment (start 122.75 73.5) (end 121.61 72.36) (width 0.762) (layer F.Cu) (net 3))
 (segment (start 122.75 99.25) (end 122.75 73.5) (width 0.762) (layer F.Cu) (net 3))
 (segment (start 121.25 100.75) (end 122.75 99.25) (width 0.762) (layer F.Cu) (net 3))
 (segment (start 88.75 100.75) (end 121.25 100.75) (width 0.762) (layer F.Cu) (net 3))
 (segment (start 86.35 98.35) (end 88.75 100.75) (width 0.762) (layer F.Cu) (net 3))
 (segment (start 85.36 88.19) (end 88.31 88.19) (width 0.762) (layer F.Cu) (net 10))
 (segment (start 100.56 77.44) (end 103.88 77.44) (width 0.762) (layer F.Cu) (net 10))
 (segment (start 97.25 80.75) (end 100.56 77.44) (width 0.762) (layer F.Cu) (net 10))
 (segment (start 95.75 80.75) (end 97.25 80.75) (width 0.762) (layer F.Cu) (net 10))
 (segment (start 88.31 88.19) (end 95.75 80.75) (width 0.762) (layer F.Cu) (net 10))
 (segment (start 85.36 85.65) (end 88.35 85.65) (width 0.762) (layer F.Cu) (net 8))
 (segment (start 97.39 72.36) (end 103.88 72.36) (width 0.762) (layer F.Cu) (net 8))
 (segment (start 97.25 72.5) (end 97.39 72.36) (width 0.762) (layer F.Cu) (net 8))
 (via (at 97.25 72.5) (size 2.54) (drill 0.8128) (layers F.Cu B.Cu) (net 8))
 (segment (start 97.25 76.75) (end 97.25 72.5) (width 0.762) (layer B.Cu) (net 8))
 (segment (start 96.75 77.25) (end 97.25 76.75) (width 0.762) (layer B.Cu) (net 8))
 (via (at 96.75 77.25) (size 2.54) (drill 0.8128) (layers F.Cu B.Cu) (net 8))
 (segment (start 88.35 85.65) (end 96.75 77.25) (width 0.762) (layer F.Cu) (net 8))
 (segment (start 119.12 85.06) (end 114.19 85.06) (width 0.762) (layer F.Cu) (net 1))
 (segment (start 86.55 72.95) (end 85.36 72.95) (width 0.762) (layer F.Cu) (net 1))
 (segment (start 89.5 70) (end 86.55 72.95) (width 0.762) (layer F.Cu) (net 1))
 (via (at 89.5 70) (size 2.54) (drill 0.8128) (layers F.Cu B.Cu) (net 1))
 (segment (start 92.5 67) (end 89.5 70) (width 0.762) (layer B.Cu) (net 1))
 (segment (start 97.5 67) (end 92.5 67) (width 0.762) (layer B.Cu) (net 1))
 (segment (start 100.5 70) (end 97.5 67) (width 0.762) (layer B.Cu) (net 1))
 (segment (start 100.5 99) (end 100.5 70) (width 0.762) (layer B.Cu) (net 1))
 (segment (start 102.25 100.75) (end 100.5 99) (width 0.762) (layer B.Cu) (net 1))
 (segment (start 108.25 100.75) (end 102.25 100.75) (width 0.762) (layer B.Cu) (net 1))
 (segment (start 112.25 96.75) (end 108.25 100.75) (width 0.762) (layer B.Cu) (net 1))
 (segment (start 112.25 87) (end 112.25 96.75) (width 0.762) (layer B.Cu) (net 1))
 (segment (start 112.5 86.75) (end 112.25 87) (width 0.762) (layer B.Cu) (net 1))
 (via (at 112.5 86.75) (size 2.54) (drill 0.8128) (layers F.Cu B.Cu) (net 1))
 (segment (start 114.19 85.06) (end 112.5 86.75) (width 0.762) (layer F.Cu) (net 1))
 (segment (start 85.36 60.25) (end 85.36 59.11) (width 0.762) (layer F.Cu) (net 14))
 (segment (start 83.75 57.5) (end 83.75 54.5) (width 0.762) (layer F.Cu) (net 14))
 (segment (start 85.36 59.11) (end 83.75 57.5) (width 0.762) (layer F.Cu) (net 14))
 (segment (start 119.12 69.82) (end 122.57 69.82) (width 0.762) (layer F.Cu) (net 4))
 (segment (start 82.52 90.73) (end 85.36 90.73) (width 0.762) (layer F.Cu) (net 4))
 (segment (start 81.5 91.75) (end 82.52 90.73) (width 0.762) (layer F.Cu) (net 4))
 (segment (start 81.5 100) (end 81.5 91.75) (width 0.762) (layer F.Cu) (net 4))
 (segment (start 83.5 102) (end 81.5 100) (width 0.762) (layer F.Cu) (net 4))
 (segment (start 122.75 102) (end 83.5 102) (width 0.762) (layer F.Cu) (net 4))
 (segment (start 124.25 100.5) (end 122.75 102) (width 0.762) (layer F.Cu) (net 4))
 (segment (start 124.25 71.5) (end 124.25 100.5) (width 0.762) (layer F.Cu) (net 4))
 (segment (start 122.57 69.82) (end 124.25 71.5) (width 0.762) (layer F.Cu) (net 4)))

